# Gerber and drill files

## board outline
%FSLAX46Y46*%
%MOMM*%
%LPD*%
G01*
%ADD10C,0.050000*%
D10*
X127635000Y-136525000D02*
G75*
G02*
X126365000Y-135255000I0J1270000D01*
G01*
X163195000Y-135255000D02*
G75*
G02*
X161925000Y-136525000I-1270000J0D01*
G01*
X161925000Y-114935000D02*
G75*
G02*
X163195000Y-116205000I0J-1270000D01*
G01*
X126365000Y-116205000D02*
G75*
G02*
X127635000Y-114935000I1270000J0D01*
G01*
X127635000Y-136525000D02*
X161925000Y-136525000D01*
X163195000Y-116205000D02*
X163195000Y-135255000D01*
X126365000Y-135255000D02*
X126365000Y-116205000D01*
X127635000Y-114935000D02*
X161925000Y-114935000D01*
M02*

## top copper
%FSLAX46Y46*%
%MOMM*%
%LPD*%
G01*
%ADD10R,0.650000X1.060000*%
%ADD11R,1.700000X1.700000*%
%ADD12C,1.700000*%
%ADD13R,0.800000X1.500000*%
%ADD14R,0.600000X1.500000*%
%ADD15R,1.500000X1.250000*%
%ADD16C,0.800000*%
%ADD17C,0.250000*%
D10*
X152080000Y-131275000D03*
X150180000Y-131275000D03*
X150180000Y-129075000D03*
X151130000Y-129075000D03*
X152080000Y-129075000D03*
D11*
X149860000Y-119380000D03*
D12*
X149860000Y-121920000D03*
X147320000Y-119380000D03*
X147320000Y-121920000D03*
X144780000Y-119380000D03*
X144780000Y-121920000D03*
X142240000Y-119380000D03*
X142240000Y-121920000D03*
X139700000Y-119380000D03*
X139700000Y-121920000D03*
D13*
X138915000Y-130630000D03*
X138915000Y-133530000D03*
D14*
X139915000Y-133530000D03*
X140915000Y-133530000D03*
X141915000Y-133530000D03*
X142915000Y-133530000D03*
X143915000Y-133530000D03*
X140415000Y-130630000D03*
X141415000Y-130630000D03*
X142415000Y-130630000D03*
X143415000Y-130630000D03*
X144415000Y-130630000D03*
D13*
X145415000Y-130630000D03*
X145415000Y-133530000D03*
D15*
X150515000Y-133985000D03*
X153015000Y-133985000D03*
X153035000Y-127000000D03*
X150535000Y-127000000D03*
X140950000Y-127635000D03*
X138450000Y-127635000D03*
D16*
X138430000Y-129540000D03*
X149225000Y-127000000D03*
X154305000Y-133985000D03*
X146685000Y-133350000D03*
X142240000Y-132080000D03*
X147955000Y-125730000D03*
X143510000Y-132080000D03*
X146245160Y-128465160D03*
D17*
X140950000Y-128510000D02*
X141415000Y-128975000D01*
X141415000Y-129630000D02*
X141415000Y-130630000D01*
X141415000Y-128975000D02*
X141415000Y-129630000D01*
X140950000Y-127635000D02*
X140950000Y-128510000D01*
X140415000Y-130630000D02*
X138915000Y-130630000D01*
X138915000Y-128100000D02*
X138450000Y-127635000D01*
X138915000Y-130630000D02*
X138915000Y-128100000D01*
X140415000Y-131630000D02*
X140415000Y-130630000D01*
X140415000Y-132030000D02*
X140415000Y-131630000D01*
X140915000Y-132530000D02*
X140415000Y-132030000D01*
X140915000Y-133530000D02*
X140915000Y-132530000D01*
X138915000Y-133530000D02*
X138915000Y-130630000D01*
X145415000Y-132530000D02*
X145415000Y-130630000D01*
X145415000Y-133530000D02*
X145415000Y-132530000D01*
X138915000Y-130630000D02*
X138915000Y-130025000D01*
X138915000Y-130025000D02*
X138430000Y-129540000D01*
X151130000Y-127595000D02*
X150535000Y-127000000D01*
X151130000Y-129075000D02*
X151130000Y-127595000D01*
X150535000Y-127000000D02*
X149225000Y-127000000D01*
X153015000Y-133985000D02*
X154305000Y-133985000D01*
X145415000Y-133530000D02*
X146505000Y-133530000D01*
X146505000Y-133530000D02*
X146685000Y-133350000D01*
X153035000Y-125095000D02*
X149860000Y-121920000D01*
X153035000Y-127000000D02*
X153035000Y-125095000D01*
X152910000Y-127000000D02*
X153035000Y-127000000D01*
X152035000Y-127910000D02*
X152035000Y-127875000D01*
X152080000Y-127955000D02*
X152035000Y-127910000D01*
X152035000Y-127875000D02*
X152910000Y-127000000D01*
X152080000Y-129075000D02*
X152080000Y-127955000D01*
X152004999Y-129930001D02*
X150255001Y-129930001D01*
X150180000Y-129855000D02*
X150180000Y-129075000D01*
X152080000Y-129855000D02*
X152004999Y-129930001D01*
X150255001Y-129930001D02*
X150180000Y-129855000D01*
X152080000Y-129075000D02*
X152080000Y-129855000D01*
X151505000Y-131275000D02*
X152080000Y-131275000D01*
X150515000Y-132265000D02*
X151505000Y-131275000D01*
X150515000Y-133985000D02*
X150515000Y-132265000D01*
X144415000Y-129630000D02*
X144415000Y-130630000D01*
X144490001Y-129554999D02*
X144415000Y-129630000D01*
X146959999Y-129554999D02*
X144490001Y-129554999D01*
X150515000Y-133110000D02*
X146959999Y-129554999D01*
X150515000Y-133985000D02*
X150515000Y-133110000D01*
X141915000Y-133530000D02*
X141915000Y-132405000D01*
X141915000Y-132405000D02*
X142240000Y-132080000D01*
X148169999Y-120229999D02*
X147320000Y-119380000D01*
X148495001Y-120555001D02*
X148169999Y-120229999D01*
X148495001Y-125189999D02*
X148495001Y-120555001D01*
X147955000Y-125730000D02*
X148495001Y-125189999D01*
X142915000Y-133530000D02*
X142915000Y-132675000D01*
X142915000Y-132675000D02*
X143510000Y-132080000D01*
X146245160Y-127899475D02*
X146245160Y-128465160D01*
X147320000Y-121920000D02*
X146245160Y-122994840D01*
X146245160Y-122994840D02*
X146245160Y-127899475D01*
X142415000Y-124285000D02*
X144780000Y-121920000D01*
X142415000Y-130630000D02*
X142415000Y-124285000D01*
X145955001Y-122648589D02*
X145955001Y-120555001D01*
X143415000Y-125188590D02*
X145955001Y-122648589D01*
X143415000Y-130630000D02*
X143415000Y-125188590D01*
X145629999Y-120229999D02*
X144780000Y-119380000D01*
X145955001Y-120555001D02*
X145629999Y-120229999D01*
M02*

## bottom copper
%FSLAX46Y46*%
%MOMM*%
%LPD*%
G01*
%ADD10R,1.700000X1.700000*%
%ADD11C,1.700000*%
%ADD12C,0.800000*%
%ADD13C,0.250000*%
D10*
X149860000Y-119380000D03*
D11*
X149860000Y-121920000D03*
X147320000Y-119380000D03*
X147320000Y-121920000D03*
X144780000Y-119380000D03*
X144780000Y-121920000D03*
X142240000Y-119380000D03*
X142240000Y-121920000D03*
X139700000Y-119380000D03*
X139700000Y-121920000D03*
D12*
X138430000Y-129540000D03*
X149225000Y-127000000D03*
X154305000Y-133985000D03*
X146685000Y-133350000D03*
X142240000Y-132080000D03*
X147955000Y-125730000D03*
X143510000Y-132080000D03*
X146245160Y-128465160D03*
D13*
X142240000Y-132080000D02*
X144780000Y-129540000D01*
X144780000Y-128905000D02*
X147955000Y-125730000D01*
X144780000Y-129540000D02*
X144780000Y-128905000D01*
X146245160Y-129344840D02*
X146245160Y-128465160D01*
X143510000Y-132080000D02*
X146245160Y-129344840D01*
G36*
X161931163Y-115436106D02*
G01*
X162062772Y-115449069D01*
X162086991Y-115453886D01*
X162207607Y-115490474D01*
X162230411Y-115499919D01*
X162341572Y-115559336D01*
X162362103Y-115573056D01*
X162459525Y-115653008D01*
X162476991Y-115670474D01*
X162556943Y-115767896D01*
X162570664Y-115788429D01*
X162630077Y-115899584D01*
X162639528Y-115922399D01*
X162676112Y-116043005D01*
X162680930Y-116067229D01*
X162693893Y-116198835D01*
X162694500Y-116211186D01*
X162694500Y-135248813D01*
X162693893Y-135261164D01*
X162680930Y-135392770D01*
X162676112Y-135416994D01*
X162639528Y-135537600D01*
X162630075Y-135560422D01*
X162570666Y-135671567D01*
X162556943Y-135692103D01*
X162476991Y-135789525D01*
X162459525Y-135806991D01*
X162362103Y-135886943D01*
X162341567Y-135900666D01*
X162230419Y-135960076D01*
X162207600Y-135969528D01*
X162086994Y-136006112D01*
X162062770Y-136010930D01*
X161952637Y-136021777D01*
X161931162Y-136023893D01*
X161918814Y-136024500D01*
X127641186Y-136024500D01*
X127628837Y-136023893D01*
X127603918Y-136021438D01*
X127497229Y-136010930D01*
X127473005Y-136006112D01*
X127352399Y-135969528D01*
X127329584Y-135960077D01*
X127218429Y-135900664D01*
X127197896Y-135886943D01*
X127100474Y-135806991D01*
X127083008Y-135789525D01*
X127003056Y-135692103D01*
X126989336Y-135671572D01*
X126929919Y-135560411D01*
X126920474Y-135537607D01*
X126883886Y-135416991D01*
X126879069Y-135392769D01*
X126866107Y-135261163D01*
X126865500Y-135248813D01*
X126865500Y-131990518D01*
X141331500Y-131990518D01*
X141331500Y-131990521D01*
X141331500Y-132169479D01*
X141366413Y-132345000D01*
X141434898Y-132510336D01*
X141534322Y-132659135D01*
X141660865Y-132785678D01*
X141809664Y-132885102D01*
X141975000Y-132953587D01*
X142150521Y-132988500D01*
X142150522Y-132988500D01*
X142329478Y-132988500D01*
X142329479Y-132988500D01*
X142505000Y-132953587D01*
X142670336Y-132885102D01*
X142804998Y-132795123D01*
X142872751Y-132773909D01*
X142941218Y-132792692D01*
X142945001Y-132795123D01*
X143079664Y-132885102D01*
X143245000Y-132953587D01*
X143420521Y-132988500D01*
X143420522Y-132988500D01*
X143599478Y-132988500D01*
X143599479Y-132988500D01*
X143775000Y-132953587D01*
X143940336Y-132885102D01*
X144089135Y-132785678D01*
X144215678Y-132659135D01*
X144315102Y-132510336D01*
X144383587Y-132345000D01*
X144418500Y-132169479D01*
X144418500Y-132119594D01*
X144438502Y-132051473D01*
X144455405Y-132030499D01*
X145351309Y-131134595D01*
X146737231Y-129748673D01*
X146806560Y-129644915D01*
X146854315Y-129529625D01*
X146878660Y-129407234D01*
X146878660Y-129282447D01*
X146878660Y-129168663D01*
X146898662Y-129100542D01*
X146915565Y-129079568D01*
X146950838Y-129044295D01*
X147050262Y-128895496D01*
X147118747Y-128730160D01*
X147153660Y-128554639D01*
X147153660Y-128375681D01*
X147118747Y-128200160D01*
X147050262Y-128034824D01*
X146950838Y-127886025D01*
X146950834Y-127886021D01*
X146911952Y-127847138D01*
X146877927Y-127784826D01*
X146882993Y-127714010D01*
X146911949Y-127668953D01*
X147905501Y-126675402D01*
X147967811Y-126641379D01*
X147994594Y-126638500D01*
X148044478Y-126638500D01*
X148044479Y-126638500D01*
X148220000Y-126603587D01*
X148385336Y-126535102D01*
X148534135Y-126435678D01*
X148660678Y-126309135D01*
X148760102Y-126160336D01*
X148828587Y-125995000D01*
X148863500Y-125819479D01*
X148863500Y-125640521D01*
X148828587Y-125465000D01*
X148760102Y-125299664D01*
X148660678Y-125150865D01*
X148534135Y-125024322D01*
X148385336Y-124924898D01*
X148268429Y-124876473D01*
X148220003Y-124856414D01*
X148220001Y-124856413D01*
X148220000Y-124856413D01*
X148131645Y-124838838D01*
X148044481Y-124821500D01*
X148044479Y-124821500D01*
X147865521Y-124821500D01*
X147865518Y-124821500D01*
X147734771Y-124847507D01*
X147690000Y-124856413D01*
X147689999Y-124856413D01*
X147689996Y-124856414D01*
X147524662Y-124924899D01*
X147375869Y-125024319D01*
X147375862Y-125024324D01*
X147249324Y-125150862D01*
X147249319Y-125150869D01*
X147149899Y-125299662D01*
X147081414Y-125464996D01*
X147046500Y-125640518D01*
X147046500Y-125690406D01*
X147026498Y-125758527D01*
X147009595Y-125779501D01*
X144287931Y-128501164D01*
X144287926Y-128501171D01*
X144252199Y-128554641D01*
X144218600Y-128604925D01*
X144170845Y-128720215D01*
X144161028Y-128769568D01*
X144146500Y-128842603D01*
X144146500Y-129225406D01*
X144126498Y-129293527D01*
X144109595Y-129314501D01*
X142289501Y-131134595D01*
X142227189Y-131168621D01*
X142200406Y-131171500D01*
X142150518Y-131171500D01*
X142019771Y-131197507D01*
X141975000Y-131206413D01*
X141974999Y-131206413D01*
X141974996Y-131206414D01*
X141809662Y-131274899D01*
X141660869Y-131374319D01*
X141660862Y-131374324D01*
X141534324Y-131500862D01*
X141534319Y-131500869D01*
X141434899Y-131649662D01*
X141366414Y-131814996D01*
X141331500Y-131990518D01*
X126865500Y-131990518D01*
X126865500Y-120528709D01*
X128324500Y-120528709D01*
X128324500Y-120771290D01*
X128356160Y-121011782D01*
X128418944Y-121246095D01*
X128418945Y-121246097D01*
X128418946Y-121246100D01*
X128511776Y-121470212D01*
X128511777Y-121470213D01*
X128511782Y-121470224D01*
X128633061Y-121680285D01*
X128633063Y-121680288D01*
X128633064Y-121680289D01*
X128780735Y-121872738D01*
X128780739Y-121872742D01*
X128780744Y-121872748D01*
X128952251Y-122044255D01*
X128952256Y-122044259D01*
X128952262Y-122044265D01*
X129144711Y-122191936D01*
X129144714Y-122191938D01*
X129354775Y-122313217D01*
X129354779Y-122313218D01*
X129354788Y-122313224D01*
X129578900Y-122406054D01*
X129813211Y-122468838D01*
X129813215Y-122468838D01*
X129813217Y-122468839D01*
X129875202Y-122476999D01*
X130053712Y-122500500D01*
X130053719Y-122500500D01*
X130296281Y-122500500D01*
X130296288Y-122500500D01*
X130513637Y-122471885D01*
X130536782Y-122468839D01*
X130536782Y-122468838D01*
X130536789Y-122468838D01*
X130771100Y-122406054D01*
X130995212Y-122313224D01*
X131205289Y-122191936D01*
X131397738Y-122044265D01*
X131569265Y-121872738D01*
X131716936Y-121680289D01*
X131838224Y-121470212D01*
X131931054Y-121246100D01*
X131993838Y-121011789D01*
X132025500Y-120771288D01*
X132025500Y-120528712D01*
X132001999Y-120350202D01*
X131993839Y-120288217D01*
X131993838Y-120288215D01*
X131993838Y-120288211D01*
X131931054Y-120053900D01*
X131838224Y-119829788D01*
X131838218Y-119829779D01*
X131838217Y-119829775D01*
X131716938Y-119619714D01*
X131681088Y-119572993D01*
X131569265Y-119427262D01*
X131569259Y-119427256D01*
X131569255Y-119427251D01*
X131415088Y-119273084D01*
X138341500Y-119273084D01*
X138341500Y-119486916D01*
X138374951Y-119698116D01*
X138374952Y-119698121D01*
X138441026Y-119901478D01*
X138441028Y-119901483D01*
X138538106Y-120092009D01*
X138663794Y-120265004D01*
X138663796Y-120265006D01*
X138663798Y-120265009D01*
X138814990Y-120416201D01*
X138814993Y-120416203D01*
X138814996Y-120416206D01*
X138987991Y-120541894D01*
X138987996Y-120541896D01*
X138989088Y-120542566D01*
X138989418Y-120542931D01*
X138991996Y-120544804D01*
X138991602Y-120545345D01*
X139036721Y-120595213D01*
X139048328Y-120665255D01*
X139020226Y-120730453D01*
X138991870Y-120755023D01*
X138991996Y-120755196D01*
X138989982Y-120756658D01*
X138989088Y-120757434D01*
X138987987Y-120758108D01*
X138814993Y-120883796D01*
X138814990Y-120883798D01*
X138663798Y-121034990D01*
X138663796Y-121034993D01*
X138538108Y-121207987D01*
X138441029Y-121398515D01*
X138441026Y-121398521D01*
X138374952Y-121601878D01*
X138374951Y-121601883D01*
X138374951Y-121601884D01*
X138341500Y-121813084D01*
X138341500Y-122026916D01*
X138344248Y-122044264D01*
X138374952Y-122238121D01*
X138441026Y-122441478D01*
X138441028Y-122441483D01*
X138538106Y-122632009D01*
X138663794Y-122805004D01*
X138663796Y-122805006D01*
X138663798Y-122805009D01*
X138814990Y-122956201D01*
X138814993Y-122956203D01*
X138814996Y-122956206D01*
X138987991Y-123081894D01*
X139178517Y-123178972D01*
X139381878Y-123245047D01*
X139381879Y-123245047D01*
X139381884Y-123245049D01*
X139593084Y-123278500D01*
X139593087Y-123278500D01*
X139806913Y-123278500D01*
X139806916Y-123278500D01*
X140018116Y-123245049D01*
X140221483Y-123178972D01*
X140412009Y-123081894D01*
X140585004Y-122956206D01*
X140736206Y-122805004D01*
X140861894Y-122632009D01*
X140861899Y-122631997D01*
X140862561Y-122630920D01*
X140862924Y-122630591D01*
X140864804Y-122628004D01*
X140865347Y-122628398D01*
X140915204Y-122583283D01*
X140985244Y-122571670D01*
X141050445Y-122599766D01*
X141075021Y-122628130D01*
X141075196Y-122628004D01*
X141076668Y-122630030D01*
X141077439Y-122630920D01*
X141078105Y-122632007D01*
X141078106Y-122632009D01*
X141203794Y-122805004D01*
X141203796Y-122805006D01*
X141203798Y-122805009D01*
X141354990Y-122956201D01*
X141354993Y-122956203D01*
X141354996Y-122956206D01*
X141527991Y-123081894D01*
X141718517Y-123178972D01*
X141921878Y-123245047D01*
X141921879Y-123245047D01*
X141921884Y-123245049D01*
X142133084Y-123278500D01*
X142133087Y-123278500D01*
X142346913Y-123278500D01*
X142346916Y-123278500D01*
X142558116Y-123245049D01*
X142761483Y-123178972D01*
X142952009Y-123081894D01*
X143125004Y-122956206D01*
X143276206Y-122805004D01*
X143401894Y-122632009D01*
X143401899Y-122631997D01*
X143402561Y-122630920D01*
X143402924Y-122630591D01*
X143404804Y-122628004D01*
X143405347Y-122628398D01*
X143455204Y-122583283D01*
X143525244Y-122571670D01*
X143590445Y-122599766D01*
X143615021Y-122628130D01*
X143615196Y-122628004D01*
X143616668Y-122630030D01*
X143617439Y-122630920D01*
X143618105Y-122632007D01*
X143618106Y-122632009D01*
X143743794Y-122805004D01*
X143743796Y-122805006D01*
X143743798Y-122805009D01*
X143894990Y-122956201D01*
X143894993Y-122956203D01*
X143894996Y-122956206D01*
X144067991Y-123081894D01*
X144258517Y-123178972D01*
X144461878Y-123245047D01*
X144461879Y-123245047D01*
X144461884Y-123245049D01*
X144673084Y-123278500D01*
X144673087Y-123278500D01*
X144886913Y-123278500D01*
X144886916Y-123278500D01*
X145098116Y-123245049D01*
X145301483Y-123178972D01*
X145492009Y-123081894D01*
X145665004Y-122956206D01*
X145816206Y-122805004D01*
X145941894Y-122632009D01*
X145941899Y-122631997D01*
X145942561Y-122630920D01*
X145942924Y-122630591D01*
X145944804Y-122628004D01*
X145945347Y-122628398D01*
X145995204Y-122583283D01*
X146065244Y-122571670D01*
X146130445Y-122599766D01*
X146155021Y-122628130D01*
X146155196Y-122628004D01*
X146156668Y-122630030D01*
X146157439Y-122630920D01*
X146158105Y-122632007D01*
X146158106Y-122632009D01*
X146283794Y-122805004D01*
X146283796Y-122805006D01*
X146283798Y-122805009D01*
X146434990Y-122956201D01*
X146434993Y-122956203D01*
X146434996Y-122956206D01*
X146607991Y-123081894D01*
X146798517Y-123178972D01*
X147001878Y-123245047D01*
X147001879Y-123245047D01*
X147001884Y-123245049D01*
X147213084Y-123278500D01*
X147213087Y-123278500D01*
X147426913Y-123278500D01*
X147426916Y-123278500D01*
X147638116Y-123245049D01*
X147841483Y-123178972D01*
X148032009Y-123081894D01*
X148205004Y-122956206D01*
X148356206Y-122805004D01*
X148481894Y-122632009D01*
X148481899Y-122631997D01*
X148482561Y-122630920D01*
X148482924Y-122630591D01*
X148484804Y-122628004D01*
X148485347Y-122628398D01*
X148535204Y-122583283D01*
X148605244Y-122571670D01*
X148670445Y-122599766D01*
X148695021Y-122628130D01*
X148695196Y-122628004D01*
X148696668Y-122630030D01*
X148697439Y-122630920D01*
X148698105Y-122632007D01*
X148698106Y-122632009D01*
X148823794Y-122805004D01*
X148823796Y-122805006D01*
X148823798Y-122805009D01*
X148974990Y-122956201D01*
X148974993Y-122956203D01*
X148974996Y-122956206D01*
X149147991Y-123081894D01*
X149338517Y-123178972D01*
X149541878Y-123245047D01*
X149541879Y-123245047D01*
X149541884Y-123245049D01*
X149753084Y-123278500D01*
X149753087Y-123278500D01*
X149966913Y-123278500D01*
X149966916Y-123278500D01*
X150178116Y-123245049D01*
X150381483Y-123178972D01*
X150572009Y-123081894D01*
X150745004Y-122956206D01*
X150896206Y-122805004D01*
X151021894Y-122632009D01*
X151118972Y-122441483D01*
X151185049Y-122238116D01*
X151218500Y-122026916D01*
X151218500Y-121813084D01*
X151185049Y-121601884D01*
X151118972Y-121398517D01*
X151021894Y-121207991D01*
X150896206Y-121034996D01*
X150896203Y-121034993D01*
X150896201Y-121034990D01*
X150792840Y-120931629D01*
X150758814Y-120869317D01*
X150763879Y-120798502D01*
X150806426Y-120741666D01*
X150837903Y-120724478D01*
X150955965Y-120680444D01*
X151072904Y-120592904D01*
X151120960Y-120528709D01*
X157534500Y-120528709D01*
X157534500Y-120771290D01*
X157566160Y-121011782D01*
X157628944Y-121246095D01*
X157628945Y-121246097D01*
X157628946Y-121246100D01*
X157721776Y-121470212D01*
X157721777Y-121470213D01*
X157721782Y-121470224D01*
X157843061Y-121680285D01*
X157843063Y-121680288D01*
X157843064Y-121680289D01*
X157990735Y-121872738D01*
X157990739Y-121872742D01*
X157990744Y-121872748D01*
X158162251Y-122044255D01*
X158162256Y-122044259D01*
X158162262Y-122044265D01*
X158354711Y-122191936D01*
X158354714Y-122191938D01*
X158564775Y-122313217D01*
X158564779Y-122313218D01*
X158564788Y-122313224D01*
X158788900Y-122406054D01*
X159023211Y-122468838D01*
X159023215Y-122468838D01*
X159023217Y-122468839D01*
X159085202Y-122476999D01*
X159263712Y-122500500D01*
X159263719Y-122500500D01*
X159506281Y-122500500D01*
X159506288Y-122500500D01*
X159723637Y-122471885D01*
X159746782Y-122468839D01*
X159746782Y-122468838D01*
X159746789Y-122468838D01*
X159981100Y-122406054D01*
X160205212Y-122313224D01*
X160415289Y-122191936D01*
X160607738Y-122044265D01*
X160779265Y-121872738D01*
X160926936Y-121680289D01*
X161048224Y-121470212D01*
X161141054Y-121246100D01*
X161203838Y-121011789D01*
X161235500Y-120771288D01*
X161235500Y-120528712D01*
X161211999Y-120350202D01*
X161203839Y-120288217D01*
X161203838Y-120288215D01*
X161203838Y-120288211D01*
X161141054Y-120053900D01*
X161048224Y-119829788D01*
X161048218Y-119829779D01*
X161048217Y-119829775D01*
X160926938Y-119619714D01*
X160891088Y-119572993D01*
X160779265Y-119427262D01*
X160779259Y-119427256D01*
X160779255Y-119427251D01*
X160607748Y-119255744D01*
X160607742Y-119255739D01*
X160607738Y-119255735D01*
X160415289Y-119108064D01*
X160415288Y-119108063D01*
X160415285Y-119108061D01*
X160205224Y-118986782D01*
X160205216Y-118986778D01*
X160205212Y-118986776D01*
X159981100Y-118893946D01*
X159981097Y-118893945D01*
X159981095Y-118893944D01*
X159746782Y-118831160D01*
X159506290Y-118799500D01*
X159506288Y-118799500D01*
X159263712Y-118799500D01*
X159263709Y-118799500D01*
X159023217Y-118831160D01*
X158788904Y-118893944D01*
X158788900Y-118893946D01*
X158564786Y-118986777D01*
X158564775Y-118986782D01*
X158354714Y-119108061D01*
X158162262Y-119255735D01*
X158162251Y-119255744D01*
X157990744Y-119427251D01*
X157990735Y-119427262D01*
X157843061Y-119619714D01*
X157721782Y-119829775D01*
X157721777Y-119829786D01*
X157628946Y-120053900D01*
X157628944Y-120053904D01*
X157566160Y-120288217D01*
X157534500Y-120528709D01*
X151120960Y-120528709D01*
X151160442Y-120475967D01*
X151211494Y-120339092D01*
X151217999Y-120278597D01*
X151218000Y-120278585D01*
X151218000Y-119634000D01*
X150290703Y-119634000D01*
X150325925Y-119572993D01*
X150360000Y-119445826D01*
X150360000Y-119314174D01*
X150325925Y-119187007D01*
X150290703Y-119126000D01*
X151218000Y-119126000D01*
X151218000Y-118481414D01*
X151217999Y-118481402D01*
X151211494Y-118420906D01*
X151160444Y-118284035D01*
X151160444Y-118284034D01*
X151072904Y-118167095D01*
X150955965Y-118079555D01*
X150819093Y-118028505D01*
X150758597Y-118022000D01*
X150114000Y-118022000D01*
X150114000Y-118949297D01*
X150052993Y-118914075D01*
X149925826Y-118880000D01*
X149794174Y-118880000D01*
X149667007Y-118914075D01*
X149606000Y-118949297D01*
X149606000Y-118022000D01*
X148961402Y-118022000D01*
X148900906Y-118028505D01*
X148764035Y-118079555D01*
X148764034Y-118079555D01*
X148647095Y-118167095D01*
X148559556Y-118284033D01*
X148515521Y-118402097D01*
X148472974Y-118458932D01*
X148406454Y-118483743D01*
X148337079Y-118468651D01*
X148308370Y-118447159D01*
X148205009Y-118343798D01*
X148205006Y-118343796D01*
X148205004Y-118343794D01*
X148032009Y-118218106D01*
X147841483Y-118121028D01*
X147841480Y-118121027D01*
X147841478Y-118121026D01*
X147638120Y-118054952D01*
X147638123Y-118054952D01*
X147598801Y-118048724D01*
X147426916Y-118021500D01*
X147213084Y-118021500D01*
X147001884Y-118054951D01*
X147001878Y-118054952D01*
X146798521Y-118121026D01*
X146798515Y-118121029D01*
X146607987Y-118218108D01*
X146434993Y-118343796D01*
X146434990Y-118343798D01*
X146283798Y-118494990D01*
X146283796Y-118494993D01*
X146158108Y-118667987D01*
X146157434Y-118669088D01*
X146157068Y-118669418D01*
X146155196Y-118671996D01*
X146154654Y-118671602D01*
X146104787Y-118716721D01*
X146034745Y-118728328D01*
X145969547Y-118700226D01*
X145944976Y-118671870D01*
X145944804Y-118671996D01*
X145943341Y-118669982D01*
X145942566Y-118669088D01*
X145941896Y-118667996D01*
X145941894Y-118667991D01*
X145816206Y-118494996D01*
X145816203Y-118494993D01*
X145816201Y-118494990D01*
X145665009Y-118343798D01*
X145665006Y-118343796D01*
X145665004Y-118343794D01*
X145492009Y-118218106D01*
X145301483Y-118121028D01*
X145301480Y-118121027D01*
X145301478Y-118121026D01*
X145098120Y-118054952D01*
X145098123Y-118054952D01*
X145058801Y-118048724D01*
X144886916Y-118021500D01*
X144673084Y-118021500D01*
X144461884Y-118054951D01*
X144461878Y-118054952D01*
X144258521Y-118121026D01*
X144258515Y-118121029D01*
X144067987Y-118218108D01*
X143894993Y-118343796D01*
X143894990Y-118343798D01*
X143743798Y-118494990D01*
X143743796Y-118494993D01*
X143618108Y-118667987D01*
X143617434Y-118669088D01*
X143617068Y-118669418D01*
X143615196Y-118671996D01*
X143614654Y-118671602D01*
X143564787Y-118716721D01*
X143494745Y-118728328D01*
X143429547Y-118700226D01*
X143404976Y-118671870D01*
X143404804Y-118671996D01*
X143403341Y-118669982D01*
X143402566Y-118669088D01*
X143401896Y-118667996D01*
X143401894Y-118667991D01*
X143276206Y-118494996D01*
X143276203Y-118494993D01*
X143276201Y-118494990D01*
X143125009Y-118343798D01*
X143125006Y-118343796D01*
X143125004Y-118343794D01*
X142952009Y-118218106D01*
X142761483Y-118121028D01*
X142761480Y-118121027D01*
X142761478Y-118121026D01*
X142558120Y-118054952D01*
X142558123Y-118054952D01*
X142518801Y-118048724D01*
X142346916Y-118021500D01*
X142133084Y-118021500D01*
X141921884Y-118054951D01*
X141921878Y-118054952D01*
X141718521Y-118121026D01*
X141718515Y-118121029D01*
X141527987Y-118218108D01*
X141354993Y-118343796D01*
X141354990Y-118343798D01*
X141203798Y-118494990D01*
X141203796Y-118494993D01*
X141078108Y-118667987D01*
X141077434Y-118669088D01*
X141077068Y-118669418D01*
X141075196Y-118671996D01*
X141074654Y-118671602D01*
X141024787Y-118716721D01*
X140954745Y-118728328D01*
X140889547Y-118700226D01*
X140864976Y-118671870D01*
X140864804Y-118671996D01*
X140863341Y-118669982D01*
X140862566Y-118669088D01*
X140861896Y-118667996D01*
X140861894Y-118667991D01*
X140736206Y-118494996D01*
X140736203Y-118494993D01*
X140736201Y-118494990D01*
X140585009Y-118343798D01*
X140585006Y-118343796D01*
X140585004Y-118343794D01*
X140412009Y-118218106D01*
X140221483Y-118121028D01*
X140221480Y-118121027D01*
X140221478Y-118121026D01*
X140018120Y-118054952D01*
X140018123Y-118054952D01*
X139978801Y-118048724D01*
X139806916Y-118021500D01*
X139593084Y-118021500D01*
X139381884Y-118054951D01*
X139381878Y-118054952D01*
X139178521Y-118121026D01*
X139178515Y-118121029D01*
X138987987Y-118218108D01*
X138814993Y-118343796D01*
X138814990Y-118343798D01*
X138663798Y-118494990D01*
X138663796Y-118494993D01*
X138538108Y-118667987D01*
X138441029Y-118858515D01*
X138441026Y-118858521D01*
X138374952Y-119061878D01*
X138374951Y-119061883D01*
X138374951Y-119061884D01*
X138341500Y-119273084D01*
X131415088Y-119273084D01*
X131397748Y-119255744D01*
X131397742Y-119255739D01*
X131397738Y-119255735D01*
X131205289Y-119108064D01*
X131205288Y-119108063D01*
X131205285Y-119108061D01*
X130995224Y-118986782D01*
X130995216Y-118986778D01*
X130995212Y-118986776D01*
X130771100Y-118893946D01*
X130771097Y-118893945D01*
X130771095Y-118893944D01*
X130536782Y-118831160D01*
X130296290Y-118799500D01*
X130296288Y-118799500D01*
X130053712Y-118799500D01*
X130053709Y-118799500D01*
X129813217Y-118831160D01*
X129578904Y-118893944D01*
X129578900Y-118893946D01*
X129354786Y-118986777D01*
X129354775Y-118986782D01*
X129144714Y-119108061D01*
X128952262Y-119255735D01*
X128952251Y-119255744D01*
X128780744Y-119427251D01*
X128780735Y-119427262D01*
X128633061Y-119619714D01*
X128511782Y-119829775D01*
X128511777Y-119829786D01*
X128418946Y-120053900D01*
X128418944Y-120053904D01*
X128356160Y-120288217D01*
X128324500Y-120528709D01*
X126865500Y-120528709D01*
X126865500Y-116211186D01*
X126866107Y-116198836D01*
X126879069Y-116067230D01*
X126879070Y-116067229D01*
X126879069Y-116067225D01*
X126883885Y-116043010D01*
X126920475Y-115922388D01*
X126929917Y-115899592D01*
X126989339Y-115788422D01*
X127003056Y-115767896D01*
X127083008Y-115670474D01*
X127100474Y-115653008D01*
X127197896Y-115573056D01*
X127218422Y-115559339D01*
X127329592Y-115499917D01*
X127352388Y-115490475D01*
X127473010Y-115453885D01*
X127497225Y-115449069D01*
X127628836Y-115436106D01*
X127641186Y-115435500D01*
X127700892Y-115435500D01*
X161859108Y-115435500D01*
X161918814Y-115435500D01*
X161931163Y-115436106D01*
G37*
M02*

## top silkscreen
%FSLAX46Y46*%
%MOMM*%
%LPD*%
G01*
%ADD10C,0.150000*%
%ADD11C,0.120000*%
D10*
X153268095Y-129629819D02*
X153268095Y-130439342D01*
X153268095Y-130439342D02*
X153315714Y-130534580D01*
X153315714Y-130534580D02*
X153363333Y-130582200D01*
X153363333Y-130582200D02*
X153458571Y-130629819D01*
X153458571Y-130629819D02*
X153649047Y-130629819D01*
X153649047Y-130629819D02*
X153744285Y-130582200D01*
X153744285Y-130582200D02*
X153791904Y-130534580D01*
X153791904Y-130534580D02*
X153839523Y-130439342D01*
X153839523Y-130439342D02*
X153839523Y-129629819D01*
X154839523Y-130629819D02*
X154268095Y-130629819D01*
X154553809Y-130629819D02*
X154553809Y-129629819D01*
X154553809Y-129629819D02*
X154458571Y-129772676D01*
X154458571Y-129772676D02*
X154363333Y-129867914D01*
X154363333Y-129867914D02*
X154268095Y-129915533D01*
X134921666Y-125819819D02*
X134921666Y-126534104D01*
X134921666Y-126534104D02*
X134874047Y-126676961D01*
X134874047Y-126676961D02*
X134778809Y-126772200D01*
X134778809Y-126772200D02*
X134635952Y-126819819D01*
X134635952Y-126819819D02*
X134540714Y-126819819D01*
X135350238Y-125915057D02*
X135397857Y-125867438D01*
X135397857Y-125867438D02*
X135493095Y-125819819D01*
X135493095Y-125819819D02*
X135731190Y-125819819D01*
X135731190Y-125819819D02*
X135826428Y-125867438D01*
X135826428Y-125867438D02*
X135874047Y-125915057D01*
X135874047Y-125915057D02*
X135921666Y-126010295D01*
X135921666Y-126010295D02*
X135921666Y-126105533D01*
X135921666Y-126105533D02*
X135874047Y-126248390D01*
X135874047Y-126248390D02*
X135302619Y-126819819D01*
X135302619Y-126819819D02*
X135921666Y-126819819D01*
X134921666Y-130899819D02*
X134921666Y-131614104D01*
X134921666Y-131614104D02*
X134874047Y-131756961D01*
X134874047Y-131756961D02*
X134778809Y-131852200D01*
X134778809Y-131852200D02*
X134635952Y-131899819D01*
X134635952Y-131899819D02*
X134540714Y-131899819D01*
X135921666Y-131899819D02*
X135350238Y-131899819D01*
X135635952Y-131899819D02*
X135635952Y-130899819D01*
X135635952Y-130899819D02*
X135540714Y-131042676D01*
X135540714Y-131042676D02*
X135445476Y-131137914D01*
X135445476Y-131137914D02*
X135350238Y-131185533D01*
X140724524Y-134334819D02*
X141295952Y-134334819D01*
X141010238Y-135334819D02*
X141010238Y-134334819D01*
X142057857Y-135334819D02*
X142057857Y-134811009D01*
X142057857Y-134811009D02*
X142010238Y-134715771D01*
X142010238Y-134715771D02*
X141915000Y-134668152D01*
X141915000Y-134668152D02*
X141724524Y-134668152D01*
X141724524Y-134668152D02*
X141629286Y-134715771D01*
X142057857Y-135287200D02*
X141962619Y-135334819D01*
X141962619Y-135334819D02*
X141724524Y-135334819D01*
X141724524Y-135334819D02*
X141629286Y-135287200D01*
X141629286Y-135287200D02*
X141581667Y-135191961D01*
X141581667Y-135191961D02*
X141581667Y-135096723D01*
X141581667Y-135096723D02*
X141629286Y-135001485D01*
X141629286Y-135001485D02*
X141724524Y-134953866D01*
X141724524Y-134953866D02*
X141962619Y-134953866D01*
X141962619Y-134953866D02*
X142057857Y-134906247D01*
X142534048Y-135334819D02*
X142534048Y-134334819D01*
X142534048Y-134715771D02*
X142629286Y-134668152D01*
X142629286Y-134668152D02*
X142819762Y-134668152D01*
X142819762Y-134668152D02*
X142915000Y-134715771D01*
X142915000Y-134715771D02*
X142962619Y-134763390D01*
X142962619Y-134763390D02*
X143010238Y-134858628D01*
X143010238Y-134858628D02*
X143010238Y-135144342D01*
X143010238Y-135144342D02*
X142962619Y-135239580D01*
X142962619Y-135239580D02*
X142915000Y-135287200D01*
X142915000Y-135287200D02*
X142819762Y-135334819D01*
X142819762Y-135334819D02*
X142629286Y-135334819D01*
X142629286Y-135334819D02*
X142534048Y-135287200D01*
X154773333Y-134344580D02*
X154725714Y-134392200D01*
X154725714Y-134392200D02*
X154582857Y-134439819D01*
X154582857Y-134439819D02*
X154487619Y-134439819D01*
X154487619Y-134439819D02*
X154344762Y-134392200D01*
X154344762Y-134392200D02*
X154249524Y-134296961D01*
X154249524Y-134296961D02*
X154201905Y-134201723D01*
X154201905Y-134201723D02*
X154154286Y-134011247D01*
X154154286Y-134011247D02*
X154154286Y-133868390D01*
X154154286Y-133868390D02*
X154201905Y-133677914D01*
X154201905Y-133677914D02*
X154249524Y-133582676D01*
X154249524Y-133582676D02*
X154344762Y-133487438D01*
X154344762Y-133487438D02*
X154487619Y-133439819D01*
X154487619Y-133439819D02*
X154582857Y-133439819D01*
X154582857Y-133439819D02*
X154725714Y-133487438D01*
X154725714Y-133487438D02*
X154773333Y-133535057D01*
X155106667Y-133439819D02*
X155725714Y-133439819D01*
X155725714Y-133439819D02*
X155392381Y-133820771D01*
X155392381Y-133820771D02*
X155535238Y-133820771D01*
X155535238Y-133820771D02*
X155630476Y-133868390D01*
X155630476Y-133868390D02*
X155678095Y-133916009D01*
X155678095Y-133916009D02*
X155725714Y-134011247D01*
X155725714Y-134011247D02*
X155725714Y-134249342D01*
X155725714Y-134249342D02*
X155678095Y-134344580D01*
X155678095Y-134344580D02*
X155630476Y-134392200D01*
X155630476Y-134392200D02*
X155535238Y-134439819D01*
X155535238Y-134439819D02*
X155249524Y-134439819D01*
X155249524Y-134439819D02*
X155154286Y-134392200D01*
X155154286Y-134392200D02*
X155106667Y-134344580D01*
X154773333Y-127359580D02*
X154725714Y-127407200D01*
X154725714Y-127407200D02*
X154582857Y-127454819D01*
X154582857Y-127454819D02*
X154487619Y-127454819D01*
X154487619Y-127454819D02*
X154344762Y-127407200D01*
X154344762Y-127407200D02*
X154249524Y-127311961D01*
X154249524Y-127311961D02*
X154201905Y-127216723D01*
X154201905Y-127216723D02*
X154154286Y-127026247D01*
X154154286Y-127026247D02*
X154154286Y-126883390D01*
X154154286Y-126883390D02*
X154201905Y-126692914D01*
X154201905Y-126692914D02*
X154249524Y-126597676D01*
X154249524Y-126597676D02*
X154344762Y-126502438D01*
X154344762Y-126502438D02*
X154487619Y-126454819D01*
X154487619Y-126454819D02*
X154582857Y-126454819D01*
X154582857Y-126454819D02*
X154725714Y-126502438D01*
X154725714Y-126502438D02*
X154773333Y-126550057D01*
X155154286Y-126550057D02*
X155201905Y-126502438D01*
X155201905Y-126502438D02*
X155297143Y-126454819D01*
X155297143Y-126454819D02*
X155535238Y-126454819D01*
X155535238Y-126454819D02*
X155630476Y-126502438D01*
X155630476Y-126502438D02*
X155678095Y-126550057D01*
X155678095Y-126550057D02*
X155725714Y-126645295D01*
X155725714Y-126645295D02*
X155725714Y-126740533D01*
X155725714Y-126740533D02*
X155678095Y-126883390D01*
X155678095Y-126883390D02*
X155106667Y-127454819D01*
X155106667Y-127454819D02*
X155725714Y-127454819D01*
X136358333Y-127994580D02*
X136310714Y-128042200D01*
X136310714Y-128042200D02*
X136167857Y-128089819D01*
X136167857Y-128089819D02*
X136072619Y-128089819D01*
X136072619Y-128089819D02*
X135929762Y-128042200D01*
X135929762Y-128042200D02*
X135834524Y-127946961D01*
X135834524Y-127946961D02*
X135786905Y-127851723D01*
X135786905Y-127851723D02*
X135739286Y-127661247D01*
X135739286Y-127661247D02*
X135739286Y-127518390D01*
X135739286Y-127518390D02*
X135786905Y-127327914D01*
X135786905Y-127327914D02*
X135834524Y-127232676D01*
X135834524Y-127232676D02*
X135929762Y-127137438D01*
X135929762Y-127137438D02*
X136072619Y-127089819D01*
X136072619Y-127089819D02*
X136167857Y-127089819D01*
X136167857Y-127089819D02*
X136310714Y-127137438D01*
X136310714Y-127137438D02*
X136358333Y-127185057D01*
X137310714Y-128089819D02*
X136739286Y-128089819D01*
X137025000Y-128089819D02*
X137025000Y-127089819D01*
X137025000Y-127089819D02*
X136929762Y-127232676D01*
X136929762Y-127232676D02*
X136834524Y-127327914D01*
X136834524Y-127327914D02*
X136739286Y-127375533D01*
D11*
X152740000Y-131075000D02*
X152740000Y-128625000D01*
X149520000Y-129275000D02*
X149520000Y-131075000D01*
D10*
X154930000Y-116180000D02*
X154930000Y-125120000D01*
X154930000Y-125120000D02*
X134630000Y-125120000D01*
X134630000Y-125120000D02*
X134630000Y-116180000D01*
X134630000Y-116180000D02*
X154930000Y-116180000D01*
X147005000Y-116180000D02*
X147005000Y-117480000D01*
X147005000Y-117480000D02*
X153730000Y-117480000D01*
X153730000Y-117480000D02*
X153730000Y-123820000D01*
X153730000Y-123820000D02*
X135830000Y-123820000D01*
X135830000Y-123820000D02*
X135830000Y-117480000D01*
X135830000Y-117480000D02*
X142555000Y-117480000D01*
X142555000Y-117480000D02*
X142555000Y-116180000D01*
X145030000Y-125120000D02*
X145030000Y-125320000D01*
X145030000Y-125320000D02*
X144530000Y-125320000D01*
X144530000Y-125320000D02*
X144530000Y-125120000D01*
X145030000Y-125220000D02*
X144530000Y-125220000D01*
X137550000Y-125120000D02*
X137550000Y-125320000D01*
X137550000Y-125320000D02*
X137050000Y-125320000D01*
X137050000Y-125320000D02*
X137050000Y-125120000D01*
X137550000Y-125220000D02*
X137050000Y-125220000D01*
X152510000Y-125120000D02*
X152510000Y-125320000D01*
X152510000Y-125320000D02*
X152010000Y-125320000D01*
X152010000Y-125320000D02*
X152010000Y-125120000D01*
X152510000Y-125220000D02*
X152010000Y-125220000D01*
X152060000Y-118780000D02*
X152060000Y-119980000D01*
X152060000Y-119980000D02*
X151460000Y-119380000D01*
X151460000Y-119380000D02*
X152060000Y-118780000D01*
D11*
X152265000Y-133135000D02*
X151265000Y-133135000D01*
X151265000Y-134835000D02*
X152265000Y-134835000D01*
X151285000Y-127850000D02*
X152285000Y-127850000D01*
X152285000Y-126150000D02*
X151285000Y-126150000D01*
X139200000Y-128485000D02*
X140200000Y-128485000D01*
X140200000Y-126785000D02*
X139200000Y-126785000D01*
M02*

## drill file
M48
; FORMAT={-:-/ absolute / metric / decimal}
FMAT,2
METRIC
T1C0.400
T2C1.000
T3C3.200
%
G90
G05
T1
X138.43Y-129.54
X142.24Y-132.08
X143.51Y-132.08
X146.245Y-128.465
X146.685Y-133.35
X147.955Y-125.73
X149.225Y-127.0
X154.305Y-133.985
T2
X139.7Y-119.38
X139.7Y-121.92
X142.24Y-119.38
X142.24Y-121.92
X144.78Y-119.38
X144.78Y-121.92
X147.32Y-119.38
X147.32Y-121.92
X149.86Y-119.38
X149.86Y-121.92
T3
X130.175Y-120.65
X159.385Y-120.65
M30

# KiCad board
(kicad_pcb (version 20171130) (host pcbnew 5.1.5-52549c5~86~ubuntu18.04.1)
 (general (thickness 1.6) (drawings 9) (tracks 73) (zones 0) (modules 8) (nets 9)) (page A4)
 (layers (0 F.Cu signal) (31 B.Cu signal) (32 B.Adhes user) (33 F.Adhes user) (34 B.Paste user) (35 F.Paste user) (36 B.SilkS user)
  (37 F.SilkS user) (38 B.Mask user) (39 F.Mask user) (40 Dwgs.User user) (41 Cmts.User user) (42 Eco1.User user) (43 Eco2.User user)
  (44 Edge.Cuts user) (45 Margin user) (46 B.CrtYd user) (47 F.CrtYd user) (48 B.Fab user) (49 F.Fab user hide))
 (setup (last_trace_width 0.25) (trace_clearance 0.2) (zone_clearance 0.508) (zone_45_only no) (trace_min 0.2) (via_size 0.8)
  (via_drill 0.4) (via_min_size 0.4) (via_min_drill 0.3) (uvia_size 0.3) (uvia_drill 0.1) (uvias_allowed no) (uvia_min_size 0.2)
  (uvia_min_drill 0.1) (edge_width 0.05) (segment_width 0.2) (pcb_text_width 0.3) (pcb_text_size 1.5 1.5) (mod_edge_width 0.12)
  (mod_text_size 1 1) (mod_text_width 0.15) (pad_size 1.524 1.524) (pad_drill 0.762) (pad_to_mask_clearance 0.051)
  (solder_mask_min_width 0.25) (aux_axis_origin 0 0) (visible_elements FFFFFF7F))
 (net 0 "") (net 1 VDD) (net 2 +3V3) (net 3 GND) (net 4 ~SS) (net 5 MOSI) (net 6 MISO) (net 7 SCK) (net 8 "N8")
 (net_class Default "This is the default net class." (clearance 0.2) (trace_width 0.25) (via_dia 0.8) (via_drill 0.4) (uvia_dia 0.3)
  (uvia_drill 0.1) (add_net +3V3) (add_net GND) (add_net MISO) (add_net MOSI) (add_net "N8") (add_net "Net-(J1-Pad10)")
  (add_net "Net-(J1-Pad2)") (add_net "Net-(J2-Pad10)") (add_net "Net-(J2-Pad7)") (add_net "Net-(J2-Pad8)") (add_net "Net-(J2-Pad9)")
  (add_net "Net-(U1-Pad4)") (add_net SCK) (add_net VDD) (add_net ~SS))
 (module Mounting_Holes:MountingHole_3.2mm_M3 (layer F.Cu) (at 159.385 120.65)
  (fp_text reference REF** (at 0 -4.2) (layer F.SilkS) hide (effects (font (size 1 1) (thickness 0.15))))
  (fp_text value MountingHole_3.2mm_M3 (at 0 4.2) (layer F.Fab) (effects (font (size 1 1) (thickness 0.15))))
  (pad 1 np_thru_hole circle (at 0 0) (size 3.2 3.2) (drill 3.2) (layers *.Cu *.Mask)))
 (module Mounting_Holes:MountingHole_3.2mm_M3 (layer F.Cu) (at 130.175 120.65)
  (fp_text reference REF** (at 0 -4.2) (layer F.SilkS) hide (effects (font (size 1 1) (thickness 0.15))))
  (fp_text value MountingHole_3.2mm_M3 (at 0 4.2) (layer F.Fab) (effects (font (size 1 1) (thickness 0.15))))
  (pad 1 np_thru_hole circle (at 0 0) (size 3.2 3.2) (drill 3.2) (layers *.Cu *.Mask)))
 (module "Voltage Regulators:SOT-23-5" (layer F.Cu) (at 151.13 130.175 270)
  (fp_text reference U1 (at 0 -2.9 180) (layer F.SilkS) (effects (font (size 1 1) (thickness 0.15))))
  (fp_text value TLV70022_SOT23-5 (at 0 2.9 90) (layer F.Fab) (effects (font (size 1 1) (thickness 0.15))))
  (fp_line (start 0.9 -1.61) (end -1.55 -1.61) (layer F.SilkS) (width 0.12))
  (fp_line (start -0.9 1.61) (end 0.9 1.61) (layer F.SilkS) (width 0.12))
  (pad 5 smd rect (at 1.1 -0.95 270) (size 1.06 0.65) (layers F.Cu F.Paste F.Mask) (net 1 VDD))
  (pad 4 smd rect (at 1.1 0.95 270) (size 1.06 0.65) (layers F.Cu F.Paste F.Mask))
  (pad 3 smd rect (at -1.1 0.95 270) (size 1.06 0.65) (layers F.Cu F.Paste F.Mask) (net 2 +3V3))
  (pad 2 smd rect (at -1.1 0 270) (size 1.06 0.65) (layers F.Cu F.Paste F.Mask) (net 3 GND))
  (pad 1 smd rect (at -1.1 -0.95 270) (size 1.06 0.65) (layers F.Cu F.Paste F.Mask) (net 2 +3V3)))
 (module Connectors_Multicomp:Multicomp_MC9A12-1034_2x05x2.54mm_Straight (layer F.Cu) (at 149.86 119.38 180)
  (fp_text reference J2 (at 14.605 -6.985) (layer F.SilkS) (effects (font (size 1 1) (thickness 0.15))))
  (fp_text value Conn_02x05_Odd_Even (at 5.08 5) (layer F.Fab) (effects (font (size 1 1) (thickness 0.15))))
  (fp_line (start -5.07 3.2) (end -5.07 -5.74) (layer F.SilkS) (width 0.15))
  (fp_line (start -5.07 -5.74) (end 15.23 -5.74) (layer F.SilkS) (width 0.15))
  (fp_line (start 15.23 -5.74) (end 15.23 3.2) (layer F.SilkS) (width 0.15))
  (fp_line (start 15.23 3.2) (end -5.07 3.2) (layer F.SilkS) (width 0.15))
  (fp_line (start 2.855 3.2) (end 2.855 1.9) (layer F.SilkS) (width 0.15))
  (fp_line (start 2.855 1.9) (end -3.87 1.9) (layer F.SilkS) (width 0.15))
  (fp_line (start -3.87 1.9) (end -3.87 -4.44) (layer F.SilkS) (width 0.15))
  (fp_line (start -3.87 -4.44) (end 14.03 -4.44) (layer F.SilkS) (width 0.15))
  (fp_line (start 14.03 -4.44) (end 14.03 1.9) (layer F.SilkS) (width 0.15))
  (fp_line (start 14.03 1.9) (end 7.305 1.9) (layer F.SilkS) (width 0.15))
  (fp_line (start 7.305 1.9) (end 7.305 3.2) (layer F.SilkS) (width 0.15))
  (fp_line (start 4.83 -5.74) (end 4.83 -5.94) (layer F.SilkS) (width 0.15))
  (fp_line (start 4.83 -5.94) (end 5.33 -5.94) (layer F.SilkS) (width 0.15))
  (fp_line (start 5.33 -5.94) (end 5.33 -5.74) (layer F.SilkS) (width 0.15))
  (fp_line (start 4.83 -5.84) (end 5.33 -5.84) (layer F.SilkS) (width 0.15))
  (fp_line (start 12.31 -5.74) (end 12.31 -5.94) (layer F.SilkS) (width 0.15))
  (fp_line (start 12.31 -5.94) (end 12.81 -5.94) (layer F.SilkS) (width 0.15))
  (fp_line (start 12.81 -5.94) (end 12.81 -5.74) (layer F.SilkS) (width 0.15))
  (fp_line (start 12.31 -5.84) (end 12.81 -5.84) (layer F.SilkS) (width 0.15))
  (fp_line (start -2.65 -5.74) (end -2.65 -5.94) (layer F.SilkS) (width 0.15))
  (fp_line (start -2.65 -5.94) (end -2.15 -5.94) (layer F.SilkS) (width 0.15))
  (fp_line (start -2.15 -5.94) (end -2.15 -5.74) (layer F.SilkS) (width 0.15))
  (fp_line (start -2.65 -5.84) (end -2.15 -5.84) (layer F.SilkS) (width 0.15))
  (fp_line (start -2.2 0.6) (end -2.2 -0.6) (layer F.SilkS) (width 0.15))
  (fp_line (start -2.2 -0.6) (end -1.6 0) (layer F.SilkS) (width 0.15))
  (fp_line (start -1.6 0) (end -2.2 0.6) (layer F.SilkS) (width 0.15))
  (pad 1 thru_hole rect (at 0 0 180) (size 1.7 1.7) (drill 1) (layers *.Cu *.Mask) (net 3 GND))
  (pad 2 thru_hole circle (at 0 -2.54 180) (size 1.7 1.7) (drill 1) (layers *.Cu *.Mask) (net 2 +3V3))
  (pad 3 thru_hole circle (at 2.54 0 180) (size 1.7 1.7) (drill 1) (layers *.Cu *.Mask) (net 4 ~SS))
  (pad 4 thru_hole circle (at 2.54 -2.54 180) (size 1.7 1.7) (drill 1) (layers *.Cu *.Mask) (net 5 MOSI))
  (pad 5 thru_hole circle (at 5.08 0 180) (size 1.7 1.7) (drill 1) (layers *.Cu *.Mask) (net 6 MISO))
  (pad 6 thru_hole circle (at 5.08 -2.54 180) (size 1.7 1.7) (drill 1) (layers *.Cu *.Mask) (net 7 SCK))
  (pad 7 thru_hole circle (at 7.62 0 180) (size 1.7 1.7) (drill 1) (layers *.Cu *.Mask))
  (pad 8 thru_hole circle (at 7.62 -2.54 180) (size 1.7 1.7) (drill 1) (layers *.Cu *.Mask))
  (pad 9 thru_hole circle (at 10.16 0 180) (size 1.7 1.7) (drill 1) (layers *.Cu *.Mask))
  (pad 10 thru_hole circle (at 10.16 -2.54 180) (size 1.7 1.7) (drill 1) (layers *.Cu *.Mask)))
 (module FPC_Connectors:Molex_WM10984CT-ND (layer F.Cu) (at 145.415 132.08 180)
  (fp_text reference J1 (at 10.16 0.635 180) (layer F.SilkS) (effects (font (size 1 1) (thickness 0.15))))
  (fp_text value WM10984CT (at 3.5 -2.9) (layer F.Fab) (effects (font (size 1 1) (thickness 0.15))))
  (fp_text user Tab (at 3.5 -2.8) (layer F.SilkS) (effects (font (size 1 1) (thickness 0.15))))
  (pad 11 smd rect (at 6.5 1.45 180) (size 0.8 1.5) (layers F.Cu F.Paste F.Mask) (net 3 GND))
  (pad 11 smd rect (at 6.5 -1.45 180) (size 0.8 1.5) (layers F.Cu F.Paste F.Mask) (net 3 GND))
  (pad 10 smd rect (at 5.5 -1.45 180) (size 0.6 1.5) (layers F.Cu F.Paste F.Mask))
  (pad 8 smd rect (at 4.5 -1.45 180) (size 0.6 1.5) (layers F.Cu F.Paste F.Mask) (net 3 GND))
  (pad 6 smd rect (at 3.5 -1.45 180) (size 0.6 1.5) (layers F.Cu F.Paste F.Mask) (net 4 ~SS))
  (pad 4 smd rect (at 2.5 -1.45 180) (size 0.6 1.5) (layers F.Cu F.Paste F.Mask) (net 5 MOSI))
  (pad 2 smd rect (at 1.5 -1.45 180) (size 0.6 1.5) (layers F.Cu F.Paste F.Mask))
  (pad 9 smd rect (at 5 1.45 180) (size 0.6 1.5) (layers F.Cu F.Paste F.Mask) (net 3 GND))
  (pad 7 smd rect (at 4 1.45 180) (size 0.6 1.5) (layers F.Cu F.Paste F.Mask) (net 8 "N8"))
  (pad 5 smd rect (at 3 1.45 180) (size 0.6 1.5) (layers F.Cu F.Paste F.Mask) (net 7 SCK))
  (pad 3 smd rect (at 2 1.45 180) (size 0.6 1.5) (layers F.Cu F.Paste F.Mask) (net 6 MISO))
  (pad 1 smd rect (at 1 1.45 180) (size 0.6 1.5) (layers F.Cu F.Paste F.Mask) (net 1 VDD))
  (pad 11 smd rect (at 0 1.45 180) (size 0.8 1.5) (layers F.Cu F.Paste F.Mask) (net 3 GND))
  (pad 11 smd rect (at 0 -1.45 180) (size 0.8 1.5) (layers F.Cu F.Paste F.Mask) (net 3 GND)))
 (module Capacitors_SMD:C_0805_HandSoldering (layer F.Cu) (at 151.765 133.985)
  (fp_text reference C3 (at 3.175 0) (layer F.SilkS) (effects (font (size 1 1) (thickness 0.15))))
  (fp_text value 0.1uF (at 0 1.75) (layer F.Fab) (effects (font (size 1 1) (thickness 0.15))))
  (fp_line (start 0.5 -0.85) (end -0.5 -0.85) (layer F.SilkS) (width 0.12))
  (fp_line (start -0.5 0.85) (end 0.5 0.85) (layer F.SilkS) (width 0.12))
  (pad 1 smd rect (at -1.25 0) (size 1.5 1.25) (layers F.Cu F.Paste F.Mask) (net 1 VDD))
  (pad 2 smd rect (at 1.25 0) (size 1.5 1.25) (layers F.Cu F.Paste F.Mask) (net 3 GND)))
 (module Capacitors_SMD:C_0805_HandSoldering (layer F.Cu) (at 151.785 127 180)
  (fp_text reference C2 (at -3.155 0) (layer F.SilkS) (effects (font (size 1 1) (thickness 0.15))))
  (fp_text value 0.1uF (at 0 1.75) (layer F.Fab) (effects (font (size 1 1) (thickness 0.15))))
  (fp_line (start 0.5 -0.85) (end -0.5 -0.85) (layer F.SilkS) (width 0.12))
  (fp_line (start -0.5 0.85) (end 0.5 0.85) (layer F.SilkS) (width 0.12))
  (pad 1 smd rect (at -1.25 0 180) (size 1.5 1.25) (layers F.Cu F.Paste F.Mask) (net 2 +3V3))
  (pad 2 smd rect (at 1.25 0 180) (size 1.5 1.25) (layers F.Cu F.Paste F.Mask) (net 3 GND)))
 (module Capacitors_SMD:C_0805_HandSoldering (layer F.Cu) (at 139.7 127.635 180)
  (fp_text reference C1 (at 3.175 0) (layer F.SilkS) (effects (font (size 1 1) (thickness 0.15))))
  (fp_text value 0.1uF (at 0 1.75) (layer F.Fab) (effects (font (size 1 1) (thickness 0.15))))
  (fp_line (start 0.5 -0.85) (end -0.5 -0.85) (layer F.SilkS) (width 0.12))
  (fp_line (start -0.5 0.85) (end 0.5 0.85) (layer F.SilkS) (width 0.12))
  (pad 1 smd rect (at -1.25 0 180) (size 1.5 1.25) (layers F.Cu F.Paste F.Mask) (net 8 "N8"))
  (pad 2 smd rect (at 1.25 0 180) (size 1.5 1.25) (layers F.Cu F.Paste F.Mask) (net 3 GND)))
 (gr_arc (start 127.635 135.255) (end 126.365 135.255) (angle -90) (layer Edge.Cuts) (width 0.05))
 (gr_arc (start 161.925 135.255) (end 161.925 136.525) (angle -90) (layer Edge.Cuts) (width 0.05))
 (gr_arc (start 161.925 116.205) (end 163.195 116.205) (angle -90) (layer Edge.Cuts) (width 0.05))
 (gr_arc (start 127.635 116.205) (end 127.635 114.935) (angle -90) (layer Edge.Cuts) (width 0.05))
 (gr_line (start 127.635 136.525) (end 161.925 136.525) (layer Edge.Cuts) (width 0.05))
 (gr_line (start 163.195 116.205) (end 163.195 135.255) (layer Edge.Cuts) (width 0.05))
 (gr_line (start 126.365 135.255) (end 126.365 116.205) (layer Edge.Cuts) (width 0.05))
 (gr_line (start 127.635 114.935) (end 161.925 114.935) (layer Edge.Cuts) (width 0.05))
 (segment (start 140.95 128.51) (end 141.415 128.975) (width 0.25) (layer F.Cu) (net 8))
 (segment (start 141.415 129.63) (end 141.415 130.63) (width 0.25) (layer F.Cu) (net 8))
 (segment (start 141.415 128.975) (end 141.415 129.63) (width 0.25) (layer F.Cu) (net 8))
 (segment (start 140.95 127.635) (end 140.95 128.51) (width 0.25) (layer F.Cu) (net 8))
 (segment (start 140.415 130.63) (end 138.915 130.63) (width 0.25) (layer F.Cu) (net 3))
 (segment (start 138.915 128.1) (end 138.45 127.635) (width 0.25) (layer F.Cu) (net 3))
 (segment (start 138.915 130.63) (end 138.915 128.1) (width 0.25) (layer F.Cu) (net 3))
 (segment (start 140.415 131.63) (end 140.415 130.63) (width 0.25) (layer F.Cu) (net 3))
 (segment (start 140.415 132.03) (end 140.415 131.63) (width 0.25) (layer F.Cu) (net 3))
 (segment (start 140.915 132.53) (end 140.415 132.03) (width 0.25) (layer F.Cu) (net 3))
 (segment (start 140.915 133.53) (end 140.915 132.53) (width 0.25) (layer F.Cu) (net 3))
 (segment (start 138.915 133.53) (end 138.915 130.63) (width 0.25) (layer F.Cu) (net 3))
 (segment (start 145.415 132.53) (end 145.415 130.63) (width 0.25) (layer F.Cu) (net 3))
 (segment (start 145.415 133.53) (end 145.415 132.53) (width 0.25) (layer F.Cu) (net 3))
 (segment (start 138.915 130.63) (end 138.915 130.025) (width 0.25) (layer F.Cu) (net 3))
 (via (at 138.43 129.54) (size 0.8) (drill 0.4) (layers F.Cu B.Cu) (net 3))
 (segment (start 138.915 130.025) (end 138.43 129.54) (width 0.25) (layer F.Cu) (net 3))
 (segment (start 151.13 127.595) (end 150.535 127) (width 0.25) (layer F.Cu) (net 3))
 (segment (start 151.13 129.075) (end 151.13 127.595) (width 0.25) (layer F.Cu) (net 3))
 (via (at 149.225 127) (size 0.8) (drill 0.4) (layers F.Cu B.Cu) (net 3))
 (segment (start 150.535 127) (end 149.225 127) (width 0.25) (layer F.Cu) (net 3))
 (via (at 154.305 133.985) (size 0.8) (drill 0.4) (layers F.Cu B.Cu) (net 3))
 (segment (start 153.015 133.985) (end 154.305 133.985) (width 0.25) (layer F.Cu) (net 3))
 (segment (start 145.415 133.53) (end 146.505 133.53) (width 0.25) (layer F.Cu) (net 3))
 (via (at 146.685 133.35) (size 0.8) (drill 0.4) (layers F.Cu B.Cu) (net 3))
 (segment (start 146.505 133.53) (end 146.685 133.35) (width 0.25) (layer F.Cu) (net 3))
 (segment (start 153.035 125.095) (end 149.86 121.92) (width 0.25) (layer F.Cu) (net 2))
 (segment (start 153.035 127) (end 153.035 125.095) (width 0.25) (layer F.Cu) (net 2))
 (segment (start 152.91 127) (end 153.035 127) (width 0.25) (layer F.Cu) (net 2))
 (segment (start 152.035 127.91) (end 152.035 127.875) (width 0.25) (layer F.Cu) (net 2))
 (segment (start 152.08 127.955) (end 152.035 127.91) (width 0.25) (layer F.Cu) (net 2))
 (segment (start 152.035 127.875) (end 152.91 127) (width 0.25) (layer F.Cu) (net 2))
 (segment (start 152.08 129.075) (end 152.08 127.955) (width 0.25) (layer F.Cu) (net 2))
 (segment (start 152.004999 129.930001) (end 150.255001 129.930001) (width 0.25) (layer F.Cu) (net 2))
 (segment (start 150.18 129.855) (end 150.18 129.075) (width 0.25) (layer F.Cu) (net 2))
 (segment (start 152.08 129.855) (end 152.004999 129.930001) (width 0.25) (layer F.Cu) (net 2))
 (segment (start 150.255001 129.930001) (end 150.18 129.855) (width 0.25) (layer F.Cu) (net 2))
 (segment (start 152.08 129.075) (end 152.08 129.855) (width 0.25) (layer F.Cu) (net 2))
 (segment (start 151.505 131.275) (end 152.08 131.275) (width 0.25) (layer F.Cu) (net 1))
 (segment (start 150.515 132.265) (end 151.505 131.275) (width 0.25) (layer F.Cu) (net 1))
 (segment (start 150.515 133.985) (end 150.515 132.265) (width 0.25) (layer F.Cu) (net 1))
 (segment (start 144.415 129.63) (end 144.415 130.63) (width 0.25) (layer F.Cu) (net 1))
 (segment (start 144.490001 129.554999) (end 144.415 129.63) (width 0.25) (layer F.Cu) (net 1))
 (segment (start 146.959999 129.554999) (end 144.490001 129.554999) (width 0.25) (layer F.Cu) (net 1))
 (segment (start 150.515 133.11) (end 146.959999 129.554999) (width 0.25) (layer F.Cu) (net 1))
 (segment (start 150.515 133.985) (end 150.515 133.11) (width 0.25) (layer F.Cu) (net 1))
 (via (at 142.24 132.08) (size 0.8) (drill 0.4) (layers F.Cu B.Cu) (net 4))
 (segment (start 141.915 133.53) (end 141.915 132.405) (width 0.25) (layer F.Cu) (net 4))
 (segment (start 141.915 132.405) (end 142.24 132.08) (width 0.25) (layer F.Cu) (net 4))
 (segment (start 142.24 132.08) (end 144.78 129.54) (width 0.25) (layer B.Cu) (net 4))
 (via (at 147.955 125.73) (size 0.8) (drill 0.4) (layers F.Cu B.Cu) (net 4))
 (segment (start 144.78 128.905) (end 147.955 125.73) (width 0.25) (layer B.Cu) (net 4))
 (segment (start 144.78 129.54) (end 144.78 128.905) (width 0.25) (layer B.Cu) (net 4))
 (segment (start 148.169999 120.229999) (end 147.32 119.38) (width 0.25) (layer F.Cu) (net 4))
 (segment (start 148.495001 120.555001) (end 148.169999 120.229999) (width 0.25) (layer F.Cu) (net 4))
 (segment (start 148.495001 125.189999) (end 148.495001 120.555001) (width 0.25) (layer F.Cu) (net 4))
 (segment (start 147.955 125.73) (end 148.495001 125.189999) (width 0.25) (layer F.Cu) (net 4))
 (via (at 143.51 132.08) (size 0.8) (drill 0.4) (layers F.Cu B.Cu) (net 5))
 (segment (start 142.915 133.53) (end 142.915 132.675) (width 0.25) (layer F.Cu) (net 5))
 (segment (start 142.915 132.675) (end 143.51 132.08) (width 0.25) (layer F.Cu) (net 5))
 (segment (start 146.24516 129.34484) (end 146.24516 128.46516) (width 0.25) (layer B.Cu) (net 5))
 (segment (start 146.24516 127.899475) (end 146.24516 128.46516) (width 0.25) (layer F.Cu) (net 5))
 (segment (start 147.32 121.92) (end 146.24516 122.99484) (width 0.25) (layer F.Cu) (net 5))
 (segment (start 143.51 132.08) (end 146.24516 129.34484) (width 0.25) (layer B.Cu) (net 5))
 (segment (start 146.24516 122.99484) (end 146.24516 127.899475) (width 0.25) (layer F.Cu) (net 5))
 (via (at 146.24516 128.46516) (size 0.8) (drill 0.4) (layers F.Cu B.Cu) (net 5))
 (segment (start 142.415 124.285) (end 144.78 121.92) (width 0.25) (layer F.Cu) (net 7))
 (segment (start 142.415 130.63) (end 142.415 124.285) (width 0.25) (layer F.Cu) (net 7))
 (segment (start 145.955001 122.648589) (end 145.955001 120.555001) (width 0.25) (layer F.Cu) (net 6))
 (segment (start 143.415 125.18859) (end 145.955001 122.648589) (width 0.25) (layer F.Cu) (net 6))
 (segment (start 143.415 130.63) (end 143.415 125.18859) (width 0.25) (layer F.Cu) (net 6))
 (segment (start 145.629999 120.229999) (end 144.78 119.38) (width 0.25) (layer F.Cu) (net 6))
 (segment (start 145.955001 120.555001) (end 145.629999 120.229999) (width 0.25) (layer F.Cu) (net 6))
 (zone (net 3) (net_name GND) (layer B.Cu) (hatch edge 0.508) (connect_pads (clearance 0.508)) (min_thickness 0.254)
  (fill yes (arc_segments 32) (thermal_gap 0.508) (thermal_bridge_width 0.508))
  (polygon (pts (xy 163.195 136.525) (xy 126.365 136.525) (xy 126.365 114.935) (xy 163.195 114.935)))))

